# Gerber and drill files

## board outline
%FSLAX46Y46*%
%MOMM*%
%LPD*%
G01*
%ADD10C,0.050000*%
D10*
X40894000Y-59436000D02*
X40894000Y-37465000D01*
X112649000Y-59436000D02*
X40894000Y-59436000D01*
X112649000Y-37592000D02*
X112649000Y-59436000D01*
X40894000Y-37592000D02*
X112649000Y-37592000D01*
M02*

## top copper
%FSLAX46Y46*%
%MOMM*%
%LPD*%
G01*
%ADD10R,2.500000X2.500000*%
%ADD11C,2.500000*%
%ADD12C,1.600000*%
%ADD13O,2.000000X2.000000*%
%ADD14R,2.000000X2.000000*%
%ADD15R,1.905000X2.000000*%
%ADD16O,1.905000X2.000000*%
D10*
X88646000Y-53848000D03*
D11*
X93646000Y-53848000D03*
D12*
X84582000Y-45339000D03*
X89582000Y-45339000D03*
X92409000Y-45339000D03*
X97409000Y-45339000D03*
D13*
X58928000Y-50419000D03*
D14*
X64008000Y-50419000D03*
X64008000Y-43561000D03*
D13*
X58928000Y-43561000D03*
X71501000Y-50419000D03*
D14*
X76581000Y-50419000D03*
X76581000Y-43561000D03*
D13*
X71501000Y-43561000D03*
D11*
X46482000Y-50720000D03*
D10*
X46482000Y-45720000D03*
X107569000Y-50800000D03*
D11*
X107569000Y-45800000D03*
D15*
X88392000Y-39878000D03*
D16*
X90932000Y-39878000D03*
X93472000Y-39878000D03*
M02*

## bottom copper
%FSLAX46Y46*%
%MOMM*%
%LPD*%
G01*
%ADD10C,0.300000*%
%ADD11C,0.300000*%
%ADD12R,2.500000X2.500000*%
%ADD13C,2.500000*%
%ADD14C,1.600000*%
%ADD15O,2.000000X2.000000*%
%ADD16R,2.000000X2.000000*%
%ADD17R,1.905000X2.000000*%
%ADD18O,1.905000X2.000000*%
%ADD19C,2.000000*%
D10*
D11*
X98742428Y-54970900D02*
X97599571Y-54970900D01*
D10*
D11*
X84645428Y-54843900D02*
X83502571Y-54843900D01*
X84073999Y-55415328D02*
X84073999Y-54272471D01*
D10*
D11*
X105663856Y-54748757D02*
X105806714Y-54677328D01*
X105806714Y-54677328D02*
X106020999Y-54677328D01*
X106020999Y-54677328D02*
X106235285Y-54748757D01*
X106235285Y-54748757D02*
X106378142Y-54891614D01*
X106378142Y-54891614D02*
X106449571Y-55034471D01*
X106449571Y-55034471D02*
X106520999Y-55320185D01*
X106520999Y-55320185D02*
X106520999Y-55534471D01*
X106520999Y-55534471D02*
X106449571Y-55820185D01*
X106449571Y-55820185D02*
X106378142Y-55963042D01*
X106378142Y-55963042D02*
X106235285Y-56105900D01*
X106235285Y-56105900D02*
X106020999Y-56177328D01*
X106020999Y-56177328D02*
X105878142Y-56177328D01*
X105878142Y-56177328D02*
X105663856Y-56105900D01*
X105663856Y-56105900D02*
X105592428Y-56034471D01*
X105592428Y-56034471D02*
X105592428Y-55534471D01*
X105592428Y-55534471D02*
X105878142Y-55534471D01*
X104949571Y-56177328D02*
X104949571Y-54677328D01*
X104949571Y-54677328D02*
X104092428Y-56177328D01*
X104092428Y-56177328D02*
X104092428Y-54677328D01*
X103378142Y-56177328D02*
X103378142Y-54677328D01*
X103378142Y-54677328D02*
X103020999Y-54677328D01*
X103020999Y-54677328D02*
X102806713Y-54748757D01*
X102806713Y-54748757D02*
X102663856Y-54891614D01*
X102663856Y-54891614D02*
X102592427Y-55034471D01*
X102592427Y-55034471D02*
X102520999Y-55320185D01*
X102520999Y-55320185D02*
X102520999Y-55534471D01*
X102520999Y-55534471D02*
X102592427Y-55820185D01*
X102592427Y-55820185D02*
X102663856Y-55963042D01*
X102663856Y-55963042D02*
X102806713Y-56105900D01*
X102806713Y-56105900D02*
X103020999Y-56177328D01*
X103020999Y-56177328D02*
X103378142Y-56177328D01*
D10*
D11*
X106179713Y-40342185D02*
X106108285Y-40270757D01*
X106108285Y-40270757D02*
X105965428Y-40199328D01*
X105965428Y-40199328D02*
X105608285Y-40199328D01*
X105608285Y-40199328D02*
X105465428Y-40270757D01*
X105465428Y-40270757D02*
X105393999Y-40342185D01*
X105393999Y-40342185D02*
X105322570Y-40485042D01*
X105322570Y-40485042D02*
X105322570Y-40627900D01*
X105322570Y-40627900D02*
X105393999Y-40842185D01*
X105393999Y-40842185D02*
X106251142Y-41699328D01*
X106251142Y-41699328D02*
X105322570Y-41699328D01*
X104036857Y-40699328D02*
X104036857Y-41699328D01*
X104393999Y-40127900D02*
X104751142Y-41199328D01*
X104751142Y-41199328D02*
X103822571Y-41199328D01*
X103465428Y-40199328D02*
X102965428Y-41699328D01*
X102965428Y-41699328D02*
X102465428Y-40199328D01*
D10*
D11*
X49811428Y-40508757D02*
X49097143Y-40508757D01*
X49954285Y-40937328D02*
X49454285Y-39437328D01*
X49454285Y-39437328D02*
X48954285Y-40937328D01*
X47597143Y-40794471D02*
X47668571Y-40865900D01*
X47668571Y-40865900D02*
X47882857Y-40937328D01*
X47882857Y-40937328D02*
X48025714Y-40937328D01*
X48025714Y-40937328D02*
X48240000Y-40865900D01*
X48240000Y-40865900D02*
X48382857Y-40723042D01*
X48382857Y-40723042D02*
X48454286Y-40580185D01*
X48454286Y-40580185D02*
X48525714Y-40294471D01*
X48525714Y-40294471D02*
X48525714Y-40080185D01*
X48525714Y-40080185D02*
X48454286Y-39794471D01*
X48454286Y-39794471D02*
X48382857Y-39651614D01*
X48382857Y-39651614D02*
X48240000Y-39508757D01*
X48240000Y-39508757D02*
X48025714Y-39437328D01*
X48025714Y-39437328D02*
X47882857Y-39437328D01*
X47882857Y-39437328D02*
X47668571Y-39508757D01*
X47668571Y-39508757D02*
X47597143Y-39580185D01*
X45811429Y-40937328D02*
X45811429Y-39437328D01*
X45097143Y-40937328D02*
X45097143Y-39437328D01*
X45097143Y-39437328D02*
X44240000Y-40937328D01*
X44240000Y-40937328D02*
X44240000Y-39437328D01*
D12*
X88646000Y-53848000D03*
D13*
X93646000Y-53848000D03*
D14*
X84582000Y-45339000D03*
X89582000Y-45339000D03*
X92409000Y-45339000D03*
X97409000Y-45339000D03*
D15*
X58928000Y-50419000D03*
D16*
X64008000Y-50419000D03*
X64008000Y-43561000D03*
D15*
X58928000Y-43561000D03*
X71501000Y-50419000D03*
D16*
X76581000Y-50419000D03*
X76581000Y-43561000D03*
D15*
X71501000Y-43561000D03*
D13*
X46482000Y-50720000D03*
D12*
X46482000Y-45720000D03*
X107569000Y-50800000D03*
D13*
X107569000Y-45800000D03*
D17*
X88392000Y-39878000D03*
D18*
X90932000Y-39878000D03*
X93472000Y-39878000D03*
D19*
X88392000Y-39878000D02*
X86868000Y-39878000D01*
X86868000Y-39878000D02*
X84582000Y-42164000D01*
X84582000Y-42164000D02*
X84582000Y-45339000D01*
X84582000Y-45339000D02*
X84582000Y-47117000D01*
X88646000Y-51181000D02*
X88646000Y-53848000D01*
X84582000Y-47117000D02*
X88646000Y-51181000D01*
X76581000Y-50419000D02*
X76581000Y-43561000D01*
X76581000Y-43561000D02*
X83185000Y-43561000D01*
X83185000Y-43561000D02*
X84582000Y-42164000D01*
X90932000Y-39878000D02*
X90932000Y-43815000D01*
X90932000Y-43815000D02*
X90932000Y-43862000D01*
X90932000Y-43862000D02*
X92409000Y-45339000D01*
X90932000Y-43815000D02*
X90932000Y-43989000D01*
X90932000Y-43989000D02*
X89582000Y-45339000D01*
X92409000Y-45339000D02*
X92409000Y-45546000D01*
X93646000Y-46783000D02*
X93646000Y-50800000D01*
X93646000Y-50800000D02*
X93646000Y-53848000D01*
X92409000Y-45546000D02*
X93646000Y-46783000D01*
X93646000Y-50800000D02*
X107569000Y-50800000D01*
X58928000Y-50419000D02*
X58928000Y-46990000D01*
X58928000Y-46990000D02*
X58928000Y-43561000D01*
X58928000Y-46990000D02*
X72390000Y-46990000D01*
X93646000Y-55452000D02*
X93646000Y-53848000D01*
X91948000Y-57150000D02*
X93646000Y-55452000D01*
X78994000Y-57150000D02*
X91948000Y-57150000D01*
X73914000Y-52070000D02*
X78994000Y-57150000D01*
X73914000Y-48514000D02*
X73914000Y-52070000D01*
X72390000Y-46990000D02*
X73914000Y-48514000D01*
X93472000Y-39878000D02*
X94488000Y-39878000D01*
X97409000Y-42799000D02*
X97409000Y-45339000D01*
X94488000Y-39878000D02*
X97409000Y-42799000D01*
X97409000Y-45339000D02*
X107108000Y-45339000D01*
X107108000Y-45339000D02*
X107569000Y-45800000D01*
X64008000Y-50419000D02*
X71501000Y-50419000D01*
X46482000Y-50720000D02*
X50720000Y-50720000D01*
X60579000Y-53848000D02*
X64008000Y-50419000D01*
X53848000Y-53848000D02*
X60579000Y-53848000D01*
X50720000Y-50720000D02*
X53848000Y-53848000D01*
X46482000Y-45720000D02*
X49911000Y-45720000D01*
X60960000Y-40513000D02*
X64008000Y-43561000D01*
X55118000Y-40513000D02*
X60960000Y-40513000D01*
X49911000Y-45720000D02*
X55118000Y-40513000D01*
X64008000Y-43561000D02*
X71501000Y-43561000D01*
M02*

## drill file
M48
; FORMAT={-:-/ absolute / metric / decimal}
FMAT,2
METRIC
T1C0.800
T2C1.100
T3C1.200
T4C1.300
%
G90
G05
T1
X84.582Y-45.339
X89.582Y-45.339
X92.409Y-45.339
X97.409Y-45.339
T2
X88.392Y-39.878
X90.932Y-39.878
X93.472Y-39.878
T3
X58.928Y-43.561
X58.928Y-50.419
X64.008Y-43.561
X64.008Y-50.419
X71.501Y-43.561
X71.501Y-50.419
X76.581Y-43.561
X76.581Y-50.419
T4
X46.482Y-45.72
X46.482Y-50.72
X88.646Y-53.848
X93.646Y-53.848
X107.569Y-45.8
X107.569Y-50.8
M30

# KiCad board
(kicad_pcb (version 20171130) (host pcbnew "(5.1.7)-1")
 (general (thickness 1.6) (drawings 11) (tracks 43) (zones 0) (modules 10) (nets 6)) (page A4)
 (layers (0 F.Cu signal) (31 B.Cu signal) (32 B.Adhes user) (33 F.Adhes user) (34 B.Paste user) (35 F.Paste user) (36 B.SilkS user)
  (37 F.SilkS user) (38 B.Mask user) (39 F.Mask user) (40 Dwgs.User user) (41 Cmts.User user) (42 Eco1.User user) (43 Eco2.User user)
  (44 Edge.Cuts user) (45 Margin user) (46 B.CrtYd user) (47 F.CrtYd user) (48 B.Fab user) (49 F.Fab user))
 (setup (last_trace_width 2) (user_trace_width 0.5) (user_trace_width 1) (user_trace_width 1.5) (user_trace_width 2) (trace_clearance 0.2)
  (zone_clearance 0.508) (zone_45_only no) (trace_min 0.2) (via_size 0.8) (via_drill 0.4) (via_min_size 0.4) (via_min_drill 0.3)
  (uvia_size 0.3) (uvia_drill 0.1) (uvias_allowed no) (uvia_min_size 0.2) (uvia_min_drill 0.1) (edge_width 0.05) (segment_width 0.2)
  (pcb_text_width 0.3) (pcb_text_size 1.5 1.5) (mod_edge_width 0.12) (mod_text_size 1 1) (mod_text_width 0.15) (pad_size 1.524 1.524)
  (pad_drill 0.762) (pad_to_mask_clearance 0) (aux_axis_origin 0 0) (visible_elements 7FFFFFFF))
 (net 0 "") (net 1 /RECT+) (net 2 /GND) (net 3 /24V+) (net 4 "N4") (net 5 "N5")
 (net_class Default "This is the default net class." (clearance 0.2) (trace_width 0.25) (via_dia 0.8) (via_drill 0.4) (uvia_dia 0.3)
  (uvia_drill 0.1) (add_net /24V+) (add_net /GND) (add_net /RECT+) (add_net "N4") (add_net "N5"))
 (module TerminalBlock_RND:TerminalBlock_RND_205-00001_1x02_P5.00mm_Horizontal (layer F.Cu) (at 88.646 53.848)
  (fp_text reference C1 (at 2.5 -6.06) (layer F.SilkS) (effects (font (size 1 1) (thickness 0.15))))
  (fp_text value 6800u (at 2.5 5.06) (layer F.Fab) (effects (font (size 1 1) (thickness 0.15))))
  (pad 1 thru_hole rect (at 0 0) (size 2.5 2.5) (drill 1.3) (layers *.Cu *.Mask) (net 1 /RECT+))
  (pad 2 thru_hole circle (at 5 0) (size 2.5 2.5) (drill 1.3) (layers *.Cu *.Mask) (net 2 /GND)))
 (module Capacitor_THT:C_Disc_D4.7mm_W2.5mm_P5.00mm (layer F.Cu) (at 84.582 45.339)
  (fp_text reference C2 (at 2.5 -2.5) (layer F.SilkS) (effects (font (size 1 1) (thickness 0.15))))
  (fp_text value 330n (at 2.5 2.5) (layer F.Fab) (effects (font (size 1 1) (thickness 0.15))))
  (pad 1 thru_hole circle (at 0 0) (size 1.6 1.6) (drill 0.8) (layers *.Cu *.Mask) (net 1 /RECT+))
  (pad 2 thru_hole circle (at 5 0) (size 1.6 1.6) (drill 0.8) (layers *.Cu *.Mask) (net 2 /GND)))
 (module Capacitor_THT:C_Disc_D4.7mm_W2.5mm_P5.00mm (layer F.Cu) (at 97.409 45.339 180)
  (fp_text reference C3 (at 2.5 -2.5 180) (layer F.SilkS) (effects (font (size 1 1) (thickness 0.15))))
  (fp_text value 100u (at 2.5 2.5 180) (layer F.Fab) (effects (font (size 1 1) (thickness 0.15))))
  (pad 2 thru_hole circle (at 5 0 180) (size 1.6 1.6) (drill 0.8) (layers *.Cu *.Mask) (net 2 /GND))
  (pad 1 thru_hole circle (at 0 0 180) (size 1.6 1.6) (drill 0.8) (layers *.Cu *.Mask) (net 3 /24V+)))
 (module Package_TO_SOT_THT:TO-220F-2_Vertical (layer F.Cu) (at 64.008 50.419 180)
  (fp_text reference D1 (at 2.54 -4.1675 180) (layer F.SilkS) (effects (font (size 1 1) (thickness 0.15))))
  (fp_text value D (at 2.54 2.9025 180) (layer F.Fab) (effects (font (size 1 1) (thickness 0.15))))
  (pad 2 thru_hole oval (at 5.08 0 180) (size 2 2) (drill 1.2) (layers *.Cu *.Mask) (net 2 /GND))
  (pad 1 thru_hole rect (at 0 0 180) (size 2 2) (drill 1.2) (layers *.Cu *.Mask) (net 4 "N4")))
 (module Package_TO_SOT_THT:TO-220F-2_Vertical (layer F.Cu) (at 64.008 43.561 180)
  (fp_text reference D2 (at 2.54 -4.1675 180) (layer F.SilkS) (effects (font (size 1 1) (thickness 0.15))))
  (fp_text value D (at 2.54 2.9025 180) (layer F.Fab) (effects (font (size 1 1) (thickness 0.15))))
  (pad 1 thru_hole rect (at 0 0 180) (size 2 2) (drill 1.2) (layers *.Cu *.Mask) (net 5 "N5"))
  (pad 2 thru_hole oval (at 5.08 0 180) (size 2 2) (drill 1.2) (layers *.Cu *.Mask) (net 2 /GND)))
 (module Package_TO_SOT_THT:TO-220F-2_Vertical (layer F.Cu) (at 76.581 50.419 180)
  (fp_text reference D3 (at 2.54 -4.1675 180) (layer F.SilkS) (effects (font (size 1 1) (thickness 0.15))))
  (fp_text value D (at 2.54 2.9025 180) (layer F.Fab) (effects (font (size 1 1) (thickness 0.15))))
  (pad 2 thru_hole oval (at 5.08 0 180) (size 2 2) (drill 1.2) (layers *.Cu *.Mask) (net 4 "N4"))
  (pad 1 thru_hole rect (at 0 0 180) (size 2 2) (drill 1.2) (layers *.Cu *.Mask) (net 1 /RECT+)))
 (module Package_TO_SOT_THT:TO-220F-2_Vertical (layer F.Cu) (at 76.581 43.561 180)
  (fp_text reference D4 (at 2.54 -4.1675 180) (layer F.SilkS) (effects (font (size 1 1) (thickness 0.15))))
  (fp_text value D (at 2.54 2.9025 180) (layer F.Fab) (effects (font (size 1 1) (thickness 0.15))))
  (pad 1 thru_hole rect (at 0 0 180) (size 2 2) (drill 1.2) (layers *.Cu *.Mask) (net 1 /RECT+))
  (pad 2 thru_hole oval (at 5.08 0 180) (size 2 2) (drill 1.2) (layers *.Cu *.Mask) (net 5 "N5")))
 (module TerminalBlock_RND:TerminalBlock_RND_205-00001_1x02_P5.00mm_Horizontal (layer F.Cu) (at 46.482 45.72 270)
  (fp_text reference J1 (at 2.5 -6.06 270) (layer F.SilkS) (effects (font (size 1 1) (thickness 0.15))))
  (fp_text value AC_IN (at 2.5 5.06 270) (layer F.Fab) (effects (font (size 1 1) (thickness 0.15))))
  (pad 2 thru_hole circle (at 5 0 270) (size 2.5 2.5) (drill 1.3) (layers *.Cu *.Mask) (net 4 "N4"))
  (pad 1 thru_hole rect (at 0 0 270) (size 2.5 2.5) (drill 1.3) (layers *.Cu *.Mask) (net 5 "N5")))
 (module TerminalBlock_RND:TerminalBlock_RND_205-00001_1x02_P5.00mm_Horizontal (layer F.Cu) (at 107.569 50.8 90)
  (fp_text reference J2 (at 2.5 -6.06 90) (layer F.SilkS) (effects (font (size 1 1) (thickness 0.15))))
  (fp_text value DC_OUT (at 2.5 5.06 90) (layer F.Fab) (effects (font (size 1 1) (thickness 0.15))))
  (pad 1 thru_hole rect (at 0 0 90) (size 2.5 2.5) (drill 1.3) (layers *.Cu *.Mask) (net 2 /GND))
  (pad 2 thru_hole circle (at 5 0 90) (size 2.5 2.5) (drill 1.3) (layers *.Cu *.Mask) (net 3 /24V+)))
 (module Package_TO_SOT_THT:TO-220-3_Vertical (layer F.Cu) (at 88.392 39.878)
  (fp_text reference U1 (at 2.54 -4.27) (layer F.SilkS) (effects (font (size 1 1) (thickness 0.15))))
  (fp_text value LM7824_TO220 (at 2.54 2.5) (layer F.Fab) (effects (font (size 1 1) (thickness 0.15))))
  (pad 1 thru_hole rect (at 0 0) (size 1.905 2) (drill 1.1) (layers *.Cu *.Mask) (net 1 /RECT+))
  (pad 2 thru_hole oval (at 2.54 0) (size 1.905 2) (drill 1.1) (layers *.Cu *.Mask) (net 2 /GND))
  (pad 3 thru_hole oval (at 5.08 0) (size 1.905 2) (drill 1.1) (layers *.Cu *.Mask) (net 3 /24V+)))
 (gr_line (start 40.894 59.436) (end 40.894 37.465) (angle 90) (layer Edge.Cuts) (width 0.05))
 (gr_line (start 112.649 59.436) (end 40.894 59.436) (angle 90) (layer Edge.Cuts) (width 0.05))
 (gr_line (start 112.649 37.592) (end 112.649 59.436) (angle 90) (layer Edge.Cuts) (width 0.05))
 (gr_line (start 40.894 37.592) (end 112.649 37.592) (angle 90) (layer Edge.Cuts) (width 0.05))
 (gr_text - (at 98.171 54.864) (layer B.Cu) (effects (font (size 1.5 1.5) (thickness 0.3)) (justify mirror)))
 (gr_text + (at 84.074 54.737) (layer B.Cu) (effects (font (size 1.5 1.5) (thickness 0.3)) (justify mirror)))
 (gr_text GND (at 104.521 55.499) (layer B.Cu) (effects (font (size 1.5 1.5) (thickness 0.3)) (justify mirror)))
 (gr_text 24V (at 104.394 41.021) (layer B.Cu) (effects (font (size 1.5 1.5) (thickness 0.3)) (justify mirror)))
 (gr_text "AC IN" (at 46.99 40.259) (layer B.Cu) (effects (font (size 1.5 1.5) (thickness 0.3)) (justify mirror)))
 (segment (start 88.392 39.878) (end 86.868 39.878) (width 2) (layer B.Cu) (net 1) (status 400000))
 (segment (start 86.868 39.878) (end 84.582 42.164) (width 2) (layer B.Cu) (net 1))
 (segment (start 84.582 42.164) (end 84.582 45.339) (width 2) (layer B.Cu) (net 1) (status 800000))
 (segment (start 84.582 45.339) (end 84.582 47.117) (width 2) (layer B.Cu) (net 1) (status 400000))
 (segment (start 88.646 51.181) (end 88.646 53.848) (width 2) (layer B.Cu) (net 1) (status 800000))
 (segment (start 84.582 47.117) (end 88.646 51.181) (width 2) (layer B.Cu) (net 1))
 (segment (start 76.581 50.419) (end 76.581 43.561) (width 2) (layer B.Cu) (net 1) (status C00000))
 (segment (start 76.581 43.561) (end 83.185 43.561) (width 2) (layer B.Cu) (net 1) (status 400000))
 (segment (start 83.185 43.561) (end 84.582 42.164) (width 2) (layer B.Cu) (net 1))
 (segment (start 90.932 39.878) (end 90.932 43.815) (width 2) (layer B.Cu) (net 2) (status 400000))
 (segment (start 90.932 43.815) (end 90.932 43.862) (width 2) (layer B.Cu) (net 2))
 (segment (start 90.932 43.862) (end 92.409 45.339) (width 2) (layer B.Cu) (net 2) (status 800000))
 (segment (start 90.932 43.815) (end 90.932 43.989) (width 2) (layer B.Cu) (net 2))
 (segment (start 90.932 43.989) (end 89.582 45.339) (width 2) (layer B.Cu) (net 2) (status 800000))
 (segment (start 92.409 45.339) (end 92.409 45.546) (width 2) (layer B.Cu) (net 2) (status C00000))
 (segment (start 93.646 46.783) (end 93.646 50.8) (width 2) (layer B.Cu) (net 2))
 (segment (start 93.646 50.8) (end 93.646 53.848) (width 2) (layer B.Cu) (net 2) (status 800000))
 (segment (start 92.409 45.546) (end 93.646 46.783) (width 2) (layer B.Cu) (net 2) (status 400000))
 (segment (start 93.646 50.8) (end 107.569 50.8) (width 2) (layer B.Cu) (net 2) (status 800000))
 (segment (start 58.928 50.419) (end 58.928 46.99) (width 2) (layer B.Cu) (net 2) (status 400000))
 (segment (start 58.928 46.99) (end 58.928 43.561) (width 2) (layer B.Cu) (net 2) (status 800000))
 (segment (start 58.928 46.99) (end 72.39 46.99) (width 2) (layer B.Cu) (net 2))
 (segment (start 93.646 55.452) (end 93.646 53.848) (width 2) (layer B.Cu) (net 2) (status 800000))
 (segment (start 91.948 57.15) (end 93.646 55.452) (width 2) (layer B.Cu) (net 2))
 (segment (start 78.994 57.15) (end 91.948 57.15) (width 2) (layer B.Cu) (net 2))
 (segment (start 73.914 52.07) (end 78.994 57.15) (width 2) (layer B.Cu) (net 2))
 (segment (start 73.914 48.514) (end 73.914 52.07) (width 2) (layer B.Cu) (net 2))
 (segment (start 72.39 46.99) (end 73.914 48.514) (width 2) (layer B.Cu) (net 2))
 (segment (start 93.472 39.878) (end 94.488 39.878) (width 2) (layer B.Cu) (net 3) (status 400000))
 (segment (start 97.409 42.799) (end 97.409 45.339) (width 2) (layer B.Cu) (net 3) (status 800000))
 (segment (start 94.488 39.878) (end 97.409 42.799) (width 2) (layer B.Cu) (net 3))
 (segment (start 97.409 45.339) (end 107.108 45.339) (width 2) (layer B.Cu) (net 3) (status C00000))
 (segment (start 107.108 45.339) (end 107.569 45.8) (width 2) (layer B.Cu) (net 3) (status C00000))
 (segment (start 64.008 50.419) (end 71.501 50.419) (width 2) (layer B.Cu) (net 4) (status C00000))
 (segment (start 46.482 50.72) (end 50.72 50.72) (width 2) (layer B.Cu) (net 4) (status 400000))
 (segment (start 60.579 53.848) (end 64.008 50.419) (width 2) (layer B.Cu) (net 4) (status 800000))
 (segment (start 53.848 53.848) (end 60.579 53.848) (width 2) (layer B.Cu) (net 4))
 (segment (start 50.72 50.72) (end 53.848 53.848) (width 2) (layer B.Cu) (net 4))
 (segment (start 46.482 45.72) (end 49.911 45.72) (width 2) (layer B.Cu) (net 5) (status 400000))
 (segment (start 60.96 40.513) (end 64.008 43.561) (width 2) (layer B.Cu) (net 5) (status 800000))
 (segment (start 55.118 40.513) (end 60.96 40.513) (width 2) (layer B.Cu) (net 5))
 (segment (start 49.911 45.72) (end 55.118 40.513) (width 2) (layer B.Cu) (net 5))
 (segment (start 64.008 43.561) (end 71.501 43.561) (width 2) (layer B.Cu) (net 5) (status C00000)))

